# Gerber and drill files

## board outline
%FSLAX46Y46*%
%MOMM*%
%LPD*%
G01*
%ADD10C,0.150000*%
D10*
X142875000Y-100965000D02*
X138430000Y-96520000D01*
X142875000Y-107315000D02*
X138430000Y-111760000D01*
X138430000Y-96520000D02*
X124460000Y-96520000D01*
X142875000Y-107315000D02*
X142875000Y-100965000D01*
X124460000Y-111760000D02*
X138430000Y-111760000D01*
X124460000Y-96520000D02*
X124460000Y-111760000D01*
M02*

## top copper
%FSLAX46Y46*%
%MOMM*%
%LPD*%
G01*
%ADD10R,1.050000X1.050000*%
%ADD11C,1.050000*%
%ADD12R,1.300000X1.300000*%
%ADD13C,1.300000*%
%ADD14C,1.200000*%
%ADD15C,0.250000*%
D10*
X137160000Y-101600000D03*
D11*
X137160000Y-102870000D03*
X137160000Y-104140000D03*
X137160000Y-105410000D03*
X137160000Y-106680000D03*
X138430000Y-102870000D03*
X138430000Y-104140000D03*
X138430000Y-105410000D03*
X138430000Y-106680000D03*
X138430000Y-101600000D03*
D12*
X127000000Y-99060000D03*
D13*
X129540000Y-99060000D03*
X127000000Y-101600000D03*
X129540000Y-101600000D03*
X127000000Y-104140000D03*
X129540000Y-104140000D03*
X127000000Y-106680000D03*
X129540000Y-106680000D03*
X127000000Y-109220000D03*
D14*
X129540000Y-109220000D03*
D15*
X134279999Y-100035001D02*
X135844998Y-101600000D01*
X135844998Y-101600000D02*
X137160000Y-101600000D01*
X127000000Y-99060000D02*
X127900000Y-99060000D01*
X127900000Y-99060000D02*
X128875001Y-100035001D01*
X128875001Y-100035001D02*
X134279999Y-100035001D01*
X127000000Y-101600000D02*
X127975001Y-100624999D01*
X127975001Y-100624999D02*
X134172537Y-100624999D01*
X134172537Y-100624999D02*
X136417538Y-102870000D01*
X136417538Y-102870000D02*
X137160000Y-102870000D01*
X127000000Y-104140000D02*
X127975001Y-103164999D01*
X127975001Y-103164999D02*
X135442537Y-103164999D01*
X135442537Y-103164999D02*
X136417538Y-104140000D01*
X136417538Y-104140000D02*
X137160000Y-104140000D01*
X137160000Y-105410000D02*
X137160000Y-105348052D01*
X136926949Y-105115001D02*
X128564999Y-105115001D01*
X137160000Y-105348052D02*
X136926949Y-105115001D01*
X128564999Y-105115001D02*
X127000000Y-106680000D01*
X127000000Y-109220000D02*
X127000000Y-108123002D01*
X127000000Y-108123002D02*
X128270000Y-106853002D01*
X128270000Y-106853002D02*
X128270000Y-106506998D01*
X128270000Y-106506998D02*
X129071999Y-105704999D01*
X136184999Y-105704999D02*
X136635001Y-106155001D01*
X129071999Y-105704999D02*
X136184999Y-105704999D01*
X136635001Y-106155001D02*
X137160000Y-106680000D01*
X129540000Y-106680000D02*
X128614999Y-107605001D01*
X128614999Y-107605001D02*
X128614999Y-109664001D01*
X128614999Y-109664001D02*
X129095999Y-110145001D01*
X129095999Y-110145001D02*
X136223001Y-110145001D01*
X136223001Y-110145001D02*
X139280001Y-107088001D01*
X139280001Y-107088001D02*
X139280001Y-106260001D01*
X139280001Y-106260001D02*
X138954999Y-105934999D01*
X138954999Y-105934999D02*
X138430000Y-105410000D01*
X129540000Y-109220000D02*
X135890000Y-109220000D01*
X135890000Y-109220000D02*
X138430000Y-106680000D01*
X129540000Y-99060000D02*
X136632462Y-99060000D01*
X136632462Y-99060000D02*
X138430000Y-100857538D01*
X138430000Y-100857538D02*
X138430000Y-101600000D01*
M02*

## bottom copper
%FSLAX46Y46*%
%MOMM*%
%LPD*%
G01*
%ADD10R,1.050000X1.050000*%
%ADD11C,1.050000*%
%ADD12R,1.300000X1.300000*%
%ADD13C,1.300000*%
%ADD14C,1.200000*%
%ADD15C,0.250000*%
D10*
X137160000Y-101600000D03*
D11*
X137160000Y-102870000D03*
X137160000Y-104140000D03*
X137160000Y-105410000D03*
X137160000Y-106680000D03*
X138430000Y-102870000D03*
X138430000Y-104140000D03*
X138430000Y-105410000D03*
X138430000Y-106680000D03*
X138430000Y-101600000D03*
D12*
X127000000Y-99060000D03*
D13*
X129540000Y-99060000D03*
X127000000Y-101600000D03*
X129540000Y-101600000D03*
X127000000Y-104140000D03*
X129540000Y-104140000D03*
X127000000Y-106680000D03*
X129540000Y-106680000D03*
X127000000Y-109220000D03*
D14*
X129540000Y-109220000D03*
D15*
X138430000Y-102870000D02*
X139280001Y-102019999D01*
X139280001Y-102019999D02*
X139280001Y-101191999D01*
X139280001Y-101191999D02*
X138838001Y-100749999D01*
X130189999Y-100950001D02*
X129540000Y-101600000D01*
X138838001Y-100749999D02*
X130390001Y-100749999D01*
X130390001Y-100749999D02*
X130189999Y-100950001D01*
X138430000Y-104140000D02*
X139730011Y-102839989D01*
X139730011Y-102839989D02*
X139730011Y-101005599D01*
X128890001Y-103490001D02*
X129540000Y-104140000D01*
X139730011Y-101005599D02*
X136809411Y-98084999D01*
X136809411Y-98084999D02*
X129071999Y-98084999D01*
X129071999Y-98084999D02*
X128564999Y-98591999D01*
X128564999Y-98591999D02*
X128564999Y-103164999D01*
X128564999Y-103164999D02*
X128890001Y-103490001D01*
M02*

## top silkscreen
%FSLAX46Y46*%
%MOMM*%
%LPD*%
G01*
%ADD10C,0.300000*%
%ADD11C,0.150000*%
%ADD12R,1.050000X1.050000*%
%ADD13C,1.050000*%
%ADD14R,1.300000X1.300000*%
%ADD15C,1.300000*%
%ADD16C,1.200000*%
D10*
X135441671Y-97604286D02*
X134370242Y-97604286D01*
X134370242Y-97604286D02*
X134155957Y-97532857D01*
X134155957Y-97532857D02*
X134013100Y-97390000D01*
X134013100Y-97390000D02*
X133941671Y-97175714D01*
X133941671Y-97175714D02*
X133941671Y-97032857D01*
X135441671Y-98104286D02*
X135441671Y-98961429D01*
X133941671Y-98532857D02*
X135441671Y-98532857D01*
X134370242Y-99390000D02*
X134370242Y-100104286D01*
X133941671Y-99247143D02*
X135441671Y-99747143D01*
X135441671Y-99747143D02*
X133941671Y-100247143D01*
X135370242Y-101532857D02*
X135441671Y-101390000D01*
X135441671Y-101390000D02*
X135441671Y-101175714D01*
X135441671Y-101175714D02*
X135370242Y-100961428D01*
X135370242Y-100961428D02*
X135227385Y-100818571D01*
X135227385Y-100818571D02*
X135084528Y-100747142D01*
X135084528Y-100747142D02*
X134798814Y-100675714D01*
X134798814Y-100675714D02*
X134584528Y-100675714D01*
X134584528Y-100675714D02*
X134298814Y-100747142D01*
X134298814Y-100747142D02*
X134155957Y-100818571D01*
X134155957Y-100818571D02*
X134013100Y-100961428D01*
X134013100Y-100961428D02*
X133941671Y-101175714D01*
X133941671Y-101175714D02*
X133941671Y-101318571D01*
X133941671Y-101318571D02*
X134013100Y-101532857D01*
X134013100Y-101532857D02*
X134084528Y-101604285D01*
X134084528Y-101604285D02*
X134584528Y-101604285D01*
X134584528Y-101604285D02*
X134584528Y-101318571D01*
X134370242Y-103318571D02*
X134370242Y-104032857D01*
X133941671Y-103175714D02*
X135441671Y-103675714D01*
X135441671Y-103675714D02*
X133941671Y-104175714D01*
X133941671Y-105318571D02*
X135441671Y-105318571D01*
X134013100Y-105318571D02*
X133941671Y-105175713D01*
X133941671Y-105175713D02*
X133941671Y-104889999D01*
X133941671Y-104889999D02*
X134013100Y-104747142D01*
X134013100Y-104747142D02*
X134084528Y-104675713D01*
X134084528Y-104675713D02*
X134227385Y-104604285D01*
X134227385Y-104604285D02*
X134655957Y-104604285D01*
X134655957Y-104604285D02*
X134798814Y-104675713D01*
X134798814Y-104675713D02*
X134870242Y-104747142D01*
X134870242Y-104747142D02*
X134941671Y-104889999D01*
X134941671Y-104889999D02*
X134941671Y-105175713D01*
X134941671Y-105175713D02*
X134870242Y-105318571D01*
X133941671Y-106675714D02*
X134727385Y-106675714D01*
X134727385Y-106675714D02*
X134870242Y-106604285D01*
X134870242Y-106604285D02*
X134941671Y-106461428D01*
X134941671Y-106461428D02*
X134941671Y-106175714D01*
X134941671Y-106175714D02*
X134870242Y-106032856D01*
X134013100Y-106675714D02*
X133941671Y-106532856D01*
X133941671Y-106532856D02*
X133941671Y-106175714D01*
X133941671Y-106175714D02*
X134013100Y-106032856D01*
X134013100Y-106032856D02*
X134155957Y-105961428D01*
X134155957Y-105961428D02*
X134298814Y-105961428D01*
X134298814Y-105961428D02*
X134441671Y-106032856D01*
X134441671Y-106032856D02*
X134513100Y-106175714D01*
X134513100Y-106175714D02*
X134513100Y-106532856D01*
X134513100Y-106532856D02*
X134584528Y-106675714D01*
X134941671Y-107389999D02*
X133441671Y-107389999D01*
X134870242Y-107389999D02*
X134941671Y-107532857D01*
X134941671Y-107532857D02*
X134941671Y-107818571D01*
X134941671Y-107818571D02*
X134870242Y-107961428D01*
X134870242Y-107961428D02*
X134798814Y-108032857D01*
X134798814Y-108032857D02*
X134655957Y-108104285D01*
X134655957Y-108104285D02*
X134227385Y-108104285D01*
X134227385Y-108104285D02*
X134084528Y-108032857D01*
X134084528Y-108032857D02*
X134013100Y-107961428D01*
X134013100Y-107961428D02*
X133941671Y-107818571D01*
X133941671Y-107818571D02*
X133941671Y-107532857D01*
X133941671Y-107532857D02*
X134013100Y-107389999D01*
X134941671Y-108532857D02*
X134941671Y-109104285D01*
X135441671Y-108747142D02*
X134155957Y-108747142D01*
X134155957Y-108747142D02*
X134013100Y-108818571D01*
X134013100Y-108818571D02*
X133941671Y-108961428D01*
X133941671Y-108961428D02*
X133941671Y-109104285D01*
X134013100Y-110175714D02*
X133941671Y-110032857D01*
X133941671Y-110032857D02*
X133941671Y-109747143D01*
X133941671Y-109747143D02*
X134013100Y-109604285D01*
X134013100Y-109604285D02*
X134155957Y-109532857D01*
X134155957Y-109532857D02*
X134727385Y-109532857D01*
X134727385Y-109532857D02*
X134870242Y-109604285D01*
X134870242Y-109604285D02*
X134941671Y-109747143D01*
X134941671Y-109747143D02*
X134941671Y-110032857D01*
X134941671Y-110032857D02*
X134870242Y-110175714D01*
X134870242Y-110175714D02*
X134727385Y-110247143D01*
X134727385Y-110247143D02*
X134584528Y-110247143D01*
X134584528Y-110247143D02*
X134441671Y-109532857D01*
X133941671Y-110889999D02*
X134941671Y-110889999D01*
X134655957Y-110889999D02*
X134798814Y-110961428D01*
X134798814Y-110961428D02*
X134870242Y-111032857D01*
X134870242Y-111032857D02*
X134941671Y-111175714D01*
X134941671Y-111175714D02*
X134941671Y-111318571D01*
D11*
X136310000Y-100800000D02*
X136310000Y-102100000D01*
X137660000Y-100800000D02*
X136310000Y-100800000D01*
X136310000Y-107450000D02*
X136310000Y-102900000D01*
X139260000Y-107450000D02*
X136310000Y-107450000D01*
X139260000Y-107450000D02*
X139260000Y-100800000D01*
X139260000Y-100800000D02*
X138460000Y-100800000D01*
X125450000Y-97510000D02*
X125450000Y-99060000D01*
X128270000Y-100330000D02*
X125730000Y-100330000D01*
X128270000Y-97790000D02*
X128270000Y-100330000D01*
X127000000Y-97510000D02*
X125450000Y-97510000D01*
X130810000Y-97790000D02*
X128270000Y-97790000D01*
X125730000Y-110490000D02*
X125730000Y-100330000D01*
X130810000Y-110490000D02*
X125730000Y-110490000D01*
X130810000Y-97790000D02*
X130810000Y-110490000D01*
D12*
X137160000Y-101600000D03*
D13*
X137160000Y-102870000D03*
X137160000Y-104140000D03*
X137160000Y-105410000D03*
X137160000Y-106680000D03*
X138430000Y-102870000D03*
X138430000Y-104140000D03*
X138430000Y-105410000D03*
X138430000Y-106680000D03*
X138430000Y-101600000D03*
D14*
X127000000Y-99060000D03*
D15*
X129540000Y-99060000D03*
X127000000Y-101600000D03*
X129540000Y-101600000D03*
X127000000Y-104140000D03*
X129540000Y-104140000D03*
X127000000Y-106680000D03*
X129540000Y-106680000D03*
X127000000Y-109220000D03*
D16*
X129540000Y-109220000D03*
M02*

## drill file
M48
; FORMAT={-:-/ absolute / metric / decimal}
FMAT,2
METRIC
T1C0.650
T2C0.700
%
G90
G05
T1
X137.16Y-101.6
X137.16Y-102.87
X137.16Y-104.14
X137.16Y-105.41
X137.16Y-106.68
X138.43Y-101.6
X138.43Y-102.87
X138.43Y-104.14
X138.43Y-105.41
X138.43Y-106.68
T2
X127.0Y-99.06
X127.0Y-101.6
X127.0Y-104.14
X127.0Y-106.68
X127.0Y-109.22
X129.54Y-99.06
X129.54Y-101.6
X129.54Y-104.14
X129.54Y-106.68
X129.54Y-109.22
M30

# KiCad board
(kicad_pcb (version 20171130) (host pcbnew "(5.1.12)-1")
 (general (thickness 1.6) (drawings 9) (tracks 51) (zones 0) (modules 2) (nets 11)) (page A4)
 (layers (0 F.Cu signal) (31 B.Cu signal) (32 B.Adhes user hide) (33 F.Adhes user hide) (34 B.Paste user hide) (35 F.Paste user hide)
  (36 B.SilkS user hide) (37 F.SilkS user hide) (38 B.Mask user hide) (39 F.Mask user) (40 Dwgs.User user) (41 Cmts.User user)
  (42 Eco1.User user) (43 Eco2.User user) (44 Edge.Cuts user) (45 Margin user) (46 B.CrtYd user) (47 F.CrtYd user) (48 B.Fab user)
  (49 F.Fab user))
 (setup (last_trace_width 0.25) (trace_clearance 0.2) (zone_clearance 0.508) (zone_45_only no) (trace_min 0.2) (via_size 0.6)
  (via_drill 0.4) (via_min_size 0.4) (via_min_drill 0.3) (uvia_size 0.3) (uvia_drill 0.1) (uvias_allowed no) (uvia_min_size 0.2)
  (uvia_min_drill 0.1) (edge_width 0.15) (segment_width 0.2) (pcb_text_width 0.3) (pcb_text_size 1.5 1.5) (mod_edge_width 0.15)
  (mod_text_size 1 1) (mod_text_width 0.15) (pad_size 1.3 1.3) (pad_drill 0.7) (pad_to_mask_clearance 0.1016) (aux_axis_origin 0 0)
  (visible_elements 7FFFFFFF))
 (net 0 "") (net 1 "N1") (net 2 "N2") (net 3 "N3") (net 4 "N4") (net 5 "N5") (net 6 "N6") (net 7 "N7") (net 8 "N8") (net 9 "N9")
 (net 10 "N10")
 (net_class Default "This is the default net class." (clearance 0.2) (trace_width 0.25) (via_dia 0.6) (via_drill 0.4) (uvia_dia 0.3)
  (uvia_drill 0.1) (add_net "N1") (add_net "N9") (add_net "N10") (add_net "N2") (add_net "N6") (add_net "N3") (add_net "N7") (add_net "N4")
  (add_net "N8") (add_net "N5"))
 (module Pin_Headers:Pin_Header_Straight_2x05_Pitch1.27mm (layer F.Cu) (at 137.16 101.6)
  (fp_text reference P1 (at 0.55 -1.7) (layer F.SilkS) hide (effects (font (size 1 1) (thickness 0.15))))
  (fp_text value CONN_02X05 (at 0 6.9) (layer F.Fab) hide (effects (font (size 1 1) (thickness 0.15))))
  (fp_line (start -0.85 -0.8) (end -0.85 0.5) (layer F.SilkS) (width 0.15))
  (fp_line (start 0.5 -0.8) (end -0.85 -0.8) (layer F.SilkS) (width 0.15))
  (fp_line (start -0.85 5.85) (end -0.85 1.3) (layer F.SilkS) (width 0.15))
  (fp_line (start 2.1 5.85) (end -0.85 5.85) (layer F.SilkS) (width 0.15))
  (fp_line (start 2.1 5.85) (end 2.1 -0.8) (layer F.SilkS) (width 0.15))
  (fp_line (start 2.1 -0.8) (end 1.3 -0.8) (layer F.SilkS) (width 0.15))
  (pad 1 thru_hole rect (at 0 0) (size 1.05 1.05) (drill 0.65) (layers *.Cu *.Mask F.SilkS) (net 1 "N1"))
  (pad 3 thru_hole circle (at 0 1.27) (size 1.05 1.05) (drill 0.65) (layers *.Cu *.Mask F.SilkS) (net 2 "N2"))
  (pad 5 thru_hole circle (at 0 2.54) (size 1.05 1.05) (drill 0.65) (layers *.Cu *.Mask F.SilkS) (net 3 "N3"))
  (pad 7 thru_hole circle (at 0 3.81) (size 1.05 1.05) (drill 0.65) (layers *.Cu *.Mask F.SilkS) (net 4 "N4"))
  (pad 9 thru_hole circle (at 0 5.08) (size 1.05 1.05) (drill 0.65) (layers *.Cu *.Mask F.SilkS) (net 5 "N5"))
  (pad 4 thru_hole circle (at 1.27 1.27) (size 1.05 1.05) (drill 0.65) (layers *.Cu *.Mask F.SilkS) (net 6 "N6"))
  (pad 6 thru_hole circle (at 1.27 2.54) (size 1.05 1.05) (drill 0.65) (layers *.Cu *.Mask F.SilkS) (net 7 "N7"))
  (pad 8 thru_hole circle (at 1.27 3.81) (size 1.05 1.05) (drill 0.65) (layers *.Cu *.Mask F.SilkS) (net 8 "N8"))
  (pad 10 thru_hole circle (at 1.27 5.08) (size 1.05 1.05) (drill 0.65) (layers *.Cu *.Mask F.SilkS) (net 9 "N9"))
  (pad 2 thru_hole circle (at 1.27 0) (size 1.05 1.05) (drill 0.65) (layers *.Cu *.Mask F.SilkS) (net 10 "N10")))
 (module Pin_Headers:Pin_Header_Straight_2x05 (layer F.Cu) (at 127 99.06)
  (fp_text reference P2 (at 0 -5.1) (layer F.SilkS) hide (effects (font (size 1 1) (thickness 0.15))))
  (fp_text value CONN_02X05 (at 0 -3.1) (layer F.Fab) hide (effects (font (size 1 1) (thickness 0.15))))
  (fp_line (start -1.55 -1.55) (end -1.55 0) (layer F.SilkS) (width 0.15))
  (fp_line (start 1.27 1.27) (end -1.27 1.27) (layer F.SilkS) (width 0.15))
  (fp_line (start 1.27 -1.27) (end 1.27 1.27) (layer F.SilkS) (width 0.15))
  (fp_line (start 0 -1.55) (end -1.55 -1.55) (layer F.SilkS) (width 0.15))
  (fp_line (start 3.81 -1.27) (end 1.27 -1.27) (layer F.SilkS) (width 0.15))
  (fp_line (start -1.27 11.43) (end -1.27 1.27) (layer F.SilkS) (width 0.15))
  (fp_line (start 3.81 11.43) (end -1.27 11.43) (layer F.SilkS) (width 0.15))
  (fp_line (start 3.81 -1.27) (end 3.81 11.43) (layer F.SilkS) (width 0.15))
  (pad 1 thru_hole rect (at 0 0) (size 1.3 1.3) (drill 0.7) (layers *.Cu *.Mask F.SilkS) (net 1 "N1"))
  (pad 2 thru_hole circle (at 2.54 0) (size 1.3 1.3) (drill 0.7) (layers *.Cu *.Mask F.SilkS) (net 10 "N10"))
  (pad 3 thru_hole circle (at 0 2.54) (size 1.3 1.3) (drill 0.7) (layers *.Cu *.Mask F.SilkS) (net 2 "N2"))
  (pad 4 thru_hole circle (at 2.54 2.54) (size 1.3 1.3) (drill 0.7) (layers *.Cu *.Mask F.SilkS) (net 6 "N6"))
  (pad 5 thru_hole circle (at 0 5.08) (size 1.3 1.3) (drill 0.7) (layers *.Cu *.Mask F.SilkS) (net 3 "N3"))
  (pad 6 thru_hole circle (at 2.54 5.08) (size 1.3 1.3) (drill 0.7) (layers *.Cu *.Mask F.SilkS) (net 7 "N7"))
  (pad 7 thru_hole circle (at 0 7.62) (size 1.3 1.3) (drill 0.7) (layers *.Cu *.Mask F.SilkS) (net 4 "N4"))
  (pad 8 thru_hole circle (at 2.54 7.62) (size 1.3 1.3) (drill 0.7) (layers *.Cu *.Mask F.SilkS) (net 8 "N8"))
  (pad 9 thru_hole circle (at 0 10.16) (size 1.3 1.3) (drill 0.7) (layers *.Cu *.Mask F.SilkS) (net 5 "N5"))
  (pad 10 thru_hole circle (at 2.54 10.16) (size 1.2 1.2) (drill 0.7) (layers *.Cu *.Mask F.SilkS) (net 9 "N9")))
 (gr_line (start 142.875 100.965) (end 138.43 96.52) (layer Edge.Cuts) (width 0.15))
 (gr_line (start 142.875 107.315) (end 138.43 111.76) (layer Edge.Cuts) (width 0.15))
 (gr_line (start 138.43 96.52) (end 124.46 96.52) (layer Edge.Cuts) (width 0.15))
 (gr_line (start 142.875 107.315) (end 142.875 100.965) (layer Edge.Cuts) (width 0.15))
 (gr_line (start 124.46 111.76) (end 138.43 111.76) (layer Edge.Cuts) (width 0.15))
 (gr_line (start 124.46 96.52) (end 124.46 111.76) (layer Edge.Cuts) (width 0.15))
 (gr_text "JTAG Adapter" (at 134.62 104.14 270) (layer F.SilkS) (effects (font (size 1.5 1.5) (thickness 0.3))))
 (segment (start 134.279999 100.035001) (end 135.844998 101.6) (width 0.25) (layer F.Cu) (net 1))
 (segment (start 135.844998 101.6) (end 137.16 101.6) (width 0.25) (layer F.Cu) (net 1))
 (segment (start 127 99.06) (end 127.9 99.06) (width 0.25) (layer F.Cu) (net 1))
 (segment (start 127.9 99.06) (end 128.875001 100.035001) (width 0.25) (layer F.Cu) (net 1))
 (segment (start 128.875001 100.035001) (end 134.279999 100.035001) (width 0.25) (layer F.Cu) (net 1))
 (segment (start 127 101.6) (end 127.975001 100.624999) (width 0.25) (layer F.Cu) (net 2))
 (segment (start 127.975001 100.624999) (end 134.172537 100.624999) (width 0.25) (layer F.Cu) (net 2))
 (segment (start 134.172537 100.624999) (end 136.417538 102.87) (width 0.25) (layer F.Cu) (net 2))
 (segment (start 136.417538 102.87) (end 137.16 102.87) (width 0.25) (layer F.Cu) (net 2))
 (segment (start 127 104.14) (end 127.975001 103.164999) (width 0.25) (layer F.Cu) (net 3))
 (segment (start 127.975001 103.164999) (end 135.442537 103.164999) (width 0.25) (layer F.Cu) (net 3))
 (segment (start 135.442537 103.164999) (end 136.417538 104.14) (width 0.25) (layer F.Cu) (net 3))
 (segment (start 136.417538 104.14) (end 137.16 104.14) (width 0.25) (layer F.Cu) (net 3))
 (segment (start 137.16 105.41) (end 137.16 105.348052) (width 0.25) (layer F.Cu) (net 4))
 (segment (start 136.926949 105.115001) (end 128.564999 105.115001) (width 0.25) (layer F.Cu) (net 4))
 (segment (start 137.16 105.348052) (end 136.926949 105.115001) (width 0.25) (layer F.Cu) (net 4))
 (segment (start 128.564999 105.115001) (end 127 106.68) (width 0.25) (layer F.Cu) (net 4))
 (segment (start 127 109.22) (end 127 108.123002) (width 0.25) (layer F.Cu) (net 5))
 (segment (start 127 108.123002) (end 128.27 106.853002) (width 0.25) (layer F.Cu) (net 5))
 (segment (start 128.27 106.853002) (end 128.27 106.506998) (width 0.25) (layer F.Cu) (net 5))
 (segment (start 128.27 106.506998) (end 129.071999 105.704999) (width 0.25) (layer F.Cu) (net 5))
 (segment (start 136.184999 105.704999) (end 136.635001 106.155001) (width 0.25) (layer F.Cu) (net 5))
 (segment (start 129.071999 105.704999) (end 136.184999 105.704999) (width 0.25) (layer F.Cu) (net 5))
 (segment (start 136.635001 106.155001) (end 137.16 106.68) (width 0.25) (layer F.Cu) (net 5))
 (segment (start 138.43 102.87) (end 139.280001 102.019999) (width 0.25) (layer B.Cu) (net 6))
 (segment (start 139.280001 102.019999) (end 139.280001 101.191999) (width 0.25) (layer B.Cu) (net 6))
 (segment (start 139.280001 101.191999) (end 138.838001 100.749999) (width 0.25) (layer B.Cu) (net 6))
 (segment (start 130.189999 100.950001) (end 129.54 101.6) (width 0.25) (layer B.Cu) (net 6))
 (segment (start 138.838001 100.749999) (end 130.390001 100.749999) (width 0.25) (layer B.Cu) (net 6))
 (segment (start 130.390001 100.749999) (end 130.189999 100.950001) (width 0.25) (layer B.Cu) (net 6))
 (segment (start 138.43 104.14) (end 139.730011 102.839989) (width 0.25) (layer B.Cu) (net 7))
 (segment (start 139.730011 102.839989) (end 139.730011 101.005599) (width 0.25) (layer B.Cu) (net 7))
 (segment (start 128.890001 103.490001) (end 129.54 104.14) (width 0.25) (layer B.Cu) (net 7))
 (segment (start 139.730011 101.005599) (end 136.809411 98.084999) (width 0.25) (layer B.Cu) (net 7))
 (segment (start 136.809411 98.084999) (end 129.071999 98.084999) (width 0.25) (layer B.Cu) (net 7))
 (segment (start 129.071999 98.084999) (end 128.564999 98.591999) (width 0.25) (layer B.Cu) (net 7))
 (segment (start 128.564999 98.591999) (end 128.564999 103.164999) (width 0.25) (layer B.Cu) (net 7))
 (segment (start 128.564999 103.164999) (end 128.890001 103.490001) (width 0.25) (layer B.Cu) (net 7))
 (segment (start 129.54 106.68) (end 128.614999 107.605001) (width 0.25) (layer F.Cu) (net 8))
 (segment (start 128.614999 107.605001) (end 128.614999 109.664001) (width 0.25) (layer F.Cu) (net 8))
 (segment (start 128.614999 109.664001) (end 129.095999 110.145001) (width 0.25) (layer F.Cu) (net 8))
 (segment (start 129.095999 110.145001) (end 136.223001 110.145001) (width 0.25) (layer F.Cu) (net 8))
 (segment (start 136.223001 110.145001) (end 139.280001 107.088001) (width 0.25) (layer F.Cu) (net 8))
 (segment (start 139.280001 107.088001) (end 139.280001 106.260001) (width 0.25) (layer F.Cu) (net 8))
 (segment (start 139.280001 106.260001) (end 138.954999 105.934999) (width 0.25) (layer F.Cu) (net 8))
 (segment (start 138.954999 105.934999) (end 138.43 105.41) (width 0.25) (layer F.Cu) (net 8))
 (segment (start 129.54 109.22) (end 135.89 109.22) (width 0.25) (layer F.Cu) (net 9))
 (segment (start 135.89 109.22) (end 138.43 106.68) (width 0.25) (layer F.Cu) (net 9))
 (segment (start 129.54 99.06) (end 136.632462 99.06) (width 0.25) (layer F.Cu) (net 10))
 (segment (start 136.632462 99.06) (end 138.43 100.857538) (width 0.25) (layer F.Cu) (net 10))
 (segment (start 138.43 100.857538) (end 138.43 101.6) (width 0.25) (layer F.Cu) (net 10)))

